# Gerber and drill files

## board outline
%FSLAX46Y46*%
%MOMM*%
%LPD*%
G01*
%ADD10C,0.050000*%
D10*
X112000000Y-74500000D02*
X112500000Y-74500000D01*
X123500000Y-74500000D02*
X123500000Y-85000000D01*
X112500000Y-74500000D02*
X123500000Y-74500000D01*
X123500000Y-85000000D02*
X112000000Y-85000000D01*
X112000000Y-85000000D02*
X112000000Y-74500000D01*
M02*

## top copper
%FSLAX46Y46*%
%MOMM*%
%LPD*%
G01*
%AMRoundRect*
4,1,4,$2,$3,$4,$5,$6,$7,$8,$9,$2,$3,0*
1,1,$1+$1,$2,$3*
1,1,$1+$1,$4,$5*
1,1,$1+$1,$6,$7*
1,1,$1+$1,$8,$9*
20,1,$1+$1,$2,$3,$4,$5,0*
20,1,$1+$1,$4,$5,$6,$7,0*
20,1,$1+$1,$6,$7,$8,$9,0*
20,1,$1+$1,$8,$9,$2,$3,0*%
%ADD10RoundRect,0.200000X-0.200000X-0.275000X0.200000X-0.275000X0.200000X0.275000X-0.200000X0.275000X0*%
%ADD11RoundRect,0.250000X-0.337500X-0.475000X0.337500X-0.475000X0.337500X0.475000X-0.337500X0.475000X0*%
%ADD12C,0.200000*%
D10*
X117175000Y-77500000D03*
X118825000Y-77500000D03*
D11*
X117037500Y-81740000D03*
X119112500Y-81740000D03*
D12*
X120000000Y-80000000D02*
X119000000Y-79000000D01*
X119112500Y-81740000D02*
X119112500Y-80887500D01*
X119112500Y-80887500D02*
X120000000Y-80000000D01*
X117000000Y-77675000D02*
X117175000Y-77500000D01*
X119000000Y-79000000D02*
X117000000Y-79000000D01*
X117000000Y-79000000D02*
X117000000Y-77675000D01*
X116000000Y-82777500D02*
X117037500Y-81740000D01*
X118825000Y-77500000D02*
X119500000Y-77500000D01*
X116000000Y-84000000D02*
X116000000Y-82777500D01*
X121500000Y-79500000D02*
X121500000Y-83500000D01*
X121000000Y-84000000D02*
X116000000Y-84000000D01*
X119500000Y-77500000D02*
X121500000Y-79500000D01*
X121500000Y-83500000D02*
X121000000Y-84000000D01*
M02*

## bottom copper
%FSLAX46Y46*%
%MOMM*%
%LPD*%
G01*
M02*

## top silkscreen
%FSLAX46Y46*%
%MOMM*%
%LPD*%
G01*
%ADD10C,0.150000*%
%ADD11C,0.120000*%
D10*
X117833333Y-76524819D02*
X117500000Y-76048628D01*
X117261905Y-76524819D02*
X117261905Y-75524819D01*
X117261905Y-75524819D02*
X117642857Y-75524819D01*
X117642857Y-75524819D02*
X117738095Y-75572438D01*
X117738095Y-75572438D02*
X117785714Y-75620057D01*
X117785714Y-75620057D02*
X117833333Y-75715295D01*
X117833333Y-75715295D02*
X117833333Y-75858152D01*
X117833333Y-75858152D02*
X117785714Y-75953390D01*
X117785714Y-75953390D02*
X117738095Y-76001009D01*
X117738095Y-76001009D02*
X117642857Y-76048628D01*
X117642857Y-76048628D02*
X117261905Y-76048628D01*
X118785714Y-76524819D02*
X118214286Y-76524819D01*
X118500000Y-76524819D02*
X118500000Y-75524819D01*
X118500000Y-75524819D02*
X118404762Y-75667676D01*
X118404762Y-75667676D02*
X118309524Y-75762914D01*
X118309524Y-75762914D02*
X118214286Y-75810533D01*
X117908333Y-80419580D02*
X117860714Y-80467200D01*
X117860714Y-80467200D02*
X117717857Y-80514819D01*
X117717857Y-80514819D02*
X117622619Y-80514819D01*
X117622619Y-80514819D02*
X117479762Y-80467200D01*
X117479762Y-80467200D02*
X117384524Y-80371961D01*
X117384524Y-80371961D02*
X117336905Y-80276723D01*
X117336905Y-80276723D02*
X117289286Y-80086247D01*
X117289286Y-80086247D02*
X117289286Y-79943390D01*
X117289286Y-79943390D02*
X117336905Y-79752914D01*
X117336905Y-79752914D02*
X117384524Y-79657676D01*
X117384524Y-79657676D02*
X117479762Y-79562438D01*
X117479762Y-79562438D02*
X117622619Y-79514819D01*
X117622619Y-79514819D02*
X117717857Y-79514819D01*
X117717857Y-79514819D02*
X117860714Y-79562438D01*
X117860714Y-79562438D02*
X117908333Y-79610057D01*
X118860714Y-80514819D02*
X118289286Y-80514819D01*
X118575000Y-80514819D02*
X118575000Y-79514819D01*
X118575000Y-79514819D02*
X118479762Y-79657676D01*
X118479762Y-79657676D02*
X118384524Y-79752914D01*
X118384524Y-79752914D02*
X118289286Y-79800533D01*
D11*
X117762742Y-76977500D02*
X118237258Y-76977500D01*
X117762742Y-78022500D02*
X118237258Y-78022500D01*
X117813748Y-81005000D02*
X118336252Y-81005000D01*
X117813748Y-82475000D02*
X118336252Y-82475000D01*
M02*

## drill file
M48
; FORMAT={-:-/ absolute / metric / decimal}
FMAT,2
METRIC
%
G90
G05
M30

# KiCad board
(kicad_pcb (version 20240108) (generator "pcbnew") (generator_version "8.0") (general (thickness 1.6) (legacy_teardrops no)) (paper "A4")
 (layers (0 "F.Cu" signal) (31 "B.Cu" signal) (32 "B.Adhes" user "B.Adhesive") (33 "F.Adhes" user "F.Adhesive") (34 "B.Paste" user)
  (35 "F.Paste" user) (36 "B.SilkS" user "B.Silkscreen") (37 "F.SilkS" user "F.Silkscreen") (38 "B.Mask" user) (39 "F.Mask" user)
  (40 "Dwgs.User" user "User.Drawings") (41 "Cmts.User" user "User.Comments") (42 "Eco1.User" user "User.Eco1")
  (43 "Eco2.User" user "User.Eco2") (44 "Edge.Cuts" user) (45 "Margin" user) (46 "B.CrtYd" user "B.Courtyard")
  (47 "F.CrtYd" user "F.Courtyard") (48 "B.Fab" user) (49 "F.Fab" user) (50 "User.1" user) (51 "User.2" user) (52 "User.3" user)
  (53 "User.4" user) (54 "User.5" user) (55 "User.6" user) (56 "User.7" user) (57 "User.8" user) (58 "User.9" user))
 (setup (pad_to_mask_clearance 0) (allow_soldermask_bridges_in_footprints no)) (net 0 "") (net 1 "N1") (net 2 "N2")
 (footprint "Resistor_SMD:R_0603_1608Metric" (layer "F.Cu") (at 118 77.5)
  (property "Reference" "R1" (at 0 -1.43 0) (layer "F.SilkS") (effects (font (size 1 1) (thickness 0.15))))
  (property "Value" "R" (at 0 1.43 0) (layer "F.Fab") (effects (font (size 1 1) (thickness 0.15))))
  (fp_line (start -0.237258 -0.5225) (end 0.237258 -0.5225) (stroke (width 0.12) (type solid)) (layer "F.SilkS"))
  (fp_line (start -0.237258 0.5225) (end 0.237258 0.5225) (stroke (width 0.12) (type solid)) (layer "F.SilkS"))
  (pad "1" smd roundrect (at -0.825 0) (size 0.8 0.95) (layers "F.Cu" "F.Paste" "F.Mask") (roundrect_rratio 0.25) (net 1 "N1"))
  (pad "2" smd roundrect (at 0.825 0) (size 0.8 0.95) (layers "F.Cu" "F.Paste" "F.Mask") (roundrect_rratio 0.25) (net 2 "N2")))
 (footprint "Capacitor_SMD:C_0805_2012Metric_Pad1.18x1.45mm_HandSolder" (layer "F.Cu") (at 118.075 81.74)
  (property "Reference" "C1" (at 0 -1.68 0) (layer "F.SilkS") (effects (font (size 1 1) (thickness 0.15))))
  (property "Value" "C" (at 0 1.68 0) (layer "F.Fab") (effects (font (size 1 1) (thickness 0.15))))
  (fp_line (start -0.261252 -0.735) (end 0.261252 -0.735) (stroke (width 0.12) (type solid)) (layer "F.SilkS"))
  (fp_line (start -0.261252 0.735) (end 0.261252 0.735) (stroke (width 0.12) (type solid)) (layer "F.SilkS"))
  (pad "1" smd roundrect (at -1.0375 0) (size 1.175 1.45) (layers "F.Cu" "F.Paste" "F.Mask") (roundrect_rratio 0.212766) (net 2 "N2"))
  (pad "2" smd roundrect (at 1.0375 0) (size 1.175 1.45) (layers "F.Cu" "F.Paste" "F.Mask") (roundrect_rratio 0.212766) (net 1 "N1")))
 (gr_line (start 112 74.5) (end 112.5 74.5) (stroke (width 0.05) (type default)) (layer "Edge.Cuts"))
 (gr_line (start 123.5 74.5) (end 123.5 85) (stroke (width 0.05) (type default)) (layer "Edge.Cuts"))
 (gr_line (start 112.5 74.5) (end 123.5 74.5) (stroke (width 0.05) (type default)) (layer "Edge.Cuts"))
 (gr_line (start 123.5 85) (end 112 85) (stroke (width 0.05) (type default)) (layer "Edge.Cuts"))
 (gr_line (start 112 85) (end 112 74.5) (stroke (width 0.05) (type default)) (layer "Edge.Cuts"))
 (segment (start 120 80) (end 119 79) (width 0.2) (layer "F.Cu") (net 1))
 (segment (start 119.1125 81.74) (end 119.1125 80.8875) (width 0.2) (layer "F.Cu") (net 1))
 (segment (start 119.1125 80.8875) (end 120 80) (width 0.2) (layer "F.Cu") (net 1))
 (segment (start 117 77.675) (end 117.175 77.5) (width 0.2) (layer "F.Cu") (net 1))
 (segment (start 119 79) (end 117 79) (width 0.2) (layer "F.Cu") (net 1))
 (segment (start 117 79) (end 117 77.675) (width 0.2) (layer "F.Cu") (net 1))
 (segment (start 116 82.7775) (end 117.0375 81.74) (width 0.2) (layer "F.Cu") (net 2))
 (segment (start 118.825 77.5) (end 119.5 77.5) (width 0.2) (layer "F.Cu") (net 2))
 (segment (start 116 84) (end 116 82.7775) (width 0.2) (layer "F.Cu") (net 2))
 (segment (start 121.5 79.5) (end 121.5 83.5) (width 0.2) (layer "F.Cu") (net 2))
 (segment (start 121 84) (end 116 84) (width 0.2) (layer "F.Cu") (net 2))
 (segment (start 119.5 77.5) (end 121.5 79.5) (width 0.2) (layer "F.Cu") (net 2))
 (segment (start 121.5 83.5) (end 121 84) (width 0.2) (layer "F.Cu") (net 2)))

